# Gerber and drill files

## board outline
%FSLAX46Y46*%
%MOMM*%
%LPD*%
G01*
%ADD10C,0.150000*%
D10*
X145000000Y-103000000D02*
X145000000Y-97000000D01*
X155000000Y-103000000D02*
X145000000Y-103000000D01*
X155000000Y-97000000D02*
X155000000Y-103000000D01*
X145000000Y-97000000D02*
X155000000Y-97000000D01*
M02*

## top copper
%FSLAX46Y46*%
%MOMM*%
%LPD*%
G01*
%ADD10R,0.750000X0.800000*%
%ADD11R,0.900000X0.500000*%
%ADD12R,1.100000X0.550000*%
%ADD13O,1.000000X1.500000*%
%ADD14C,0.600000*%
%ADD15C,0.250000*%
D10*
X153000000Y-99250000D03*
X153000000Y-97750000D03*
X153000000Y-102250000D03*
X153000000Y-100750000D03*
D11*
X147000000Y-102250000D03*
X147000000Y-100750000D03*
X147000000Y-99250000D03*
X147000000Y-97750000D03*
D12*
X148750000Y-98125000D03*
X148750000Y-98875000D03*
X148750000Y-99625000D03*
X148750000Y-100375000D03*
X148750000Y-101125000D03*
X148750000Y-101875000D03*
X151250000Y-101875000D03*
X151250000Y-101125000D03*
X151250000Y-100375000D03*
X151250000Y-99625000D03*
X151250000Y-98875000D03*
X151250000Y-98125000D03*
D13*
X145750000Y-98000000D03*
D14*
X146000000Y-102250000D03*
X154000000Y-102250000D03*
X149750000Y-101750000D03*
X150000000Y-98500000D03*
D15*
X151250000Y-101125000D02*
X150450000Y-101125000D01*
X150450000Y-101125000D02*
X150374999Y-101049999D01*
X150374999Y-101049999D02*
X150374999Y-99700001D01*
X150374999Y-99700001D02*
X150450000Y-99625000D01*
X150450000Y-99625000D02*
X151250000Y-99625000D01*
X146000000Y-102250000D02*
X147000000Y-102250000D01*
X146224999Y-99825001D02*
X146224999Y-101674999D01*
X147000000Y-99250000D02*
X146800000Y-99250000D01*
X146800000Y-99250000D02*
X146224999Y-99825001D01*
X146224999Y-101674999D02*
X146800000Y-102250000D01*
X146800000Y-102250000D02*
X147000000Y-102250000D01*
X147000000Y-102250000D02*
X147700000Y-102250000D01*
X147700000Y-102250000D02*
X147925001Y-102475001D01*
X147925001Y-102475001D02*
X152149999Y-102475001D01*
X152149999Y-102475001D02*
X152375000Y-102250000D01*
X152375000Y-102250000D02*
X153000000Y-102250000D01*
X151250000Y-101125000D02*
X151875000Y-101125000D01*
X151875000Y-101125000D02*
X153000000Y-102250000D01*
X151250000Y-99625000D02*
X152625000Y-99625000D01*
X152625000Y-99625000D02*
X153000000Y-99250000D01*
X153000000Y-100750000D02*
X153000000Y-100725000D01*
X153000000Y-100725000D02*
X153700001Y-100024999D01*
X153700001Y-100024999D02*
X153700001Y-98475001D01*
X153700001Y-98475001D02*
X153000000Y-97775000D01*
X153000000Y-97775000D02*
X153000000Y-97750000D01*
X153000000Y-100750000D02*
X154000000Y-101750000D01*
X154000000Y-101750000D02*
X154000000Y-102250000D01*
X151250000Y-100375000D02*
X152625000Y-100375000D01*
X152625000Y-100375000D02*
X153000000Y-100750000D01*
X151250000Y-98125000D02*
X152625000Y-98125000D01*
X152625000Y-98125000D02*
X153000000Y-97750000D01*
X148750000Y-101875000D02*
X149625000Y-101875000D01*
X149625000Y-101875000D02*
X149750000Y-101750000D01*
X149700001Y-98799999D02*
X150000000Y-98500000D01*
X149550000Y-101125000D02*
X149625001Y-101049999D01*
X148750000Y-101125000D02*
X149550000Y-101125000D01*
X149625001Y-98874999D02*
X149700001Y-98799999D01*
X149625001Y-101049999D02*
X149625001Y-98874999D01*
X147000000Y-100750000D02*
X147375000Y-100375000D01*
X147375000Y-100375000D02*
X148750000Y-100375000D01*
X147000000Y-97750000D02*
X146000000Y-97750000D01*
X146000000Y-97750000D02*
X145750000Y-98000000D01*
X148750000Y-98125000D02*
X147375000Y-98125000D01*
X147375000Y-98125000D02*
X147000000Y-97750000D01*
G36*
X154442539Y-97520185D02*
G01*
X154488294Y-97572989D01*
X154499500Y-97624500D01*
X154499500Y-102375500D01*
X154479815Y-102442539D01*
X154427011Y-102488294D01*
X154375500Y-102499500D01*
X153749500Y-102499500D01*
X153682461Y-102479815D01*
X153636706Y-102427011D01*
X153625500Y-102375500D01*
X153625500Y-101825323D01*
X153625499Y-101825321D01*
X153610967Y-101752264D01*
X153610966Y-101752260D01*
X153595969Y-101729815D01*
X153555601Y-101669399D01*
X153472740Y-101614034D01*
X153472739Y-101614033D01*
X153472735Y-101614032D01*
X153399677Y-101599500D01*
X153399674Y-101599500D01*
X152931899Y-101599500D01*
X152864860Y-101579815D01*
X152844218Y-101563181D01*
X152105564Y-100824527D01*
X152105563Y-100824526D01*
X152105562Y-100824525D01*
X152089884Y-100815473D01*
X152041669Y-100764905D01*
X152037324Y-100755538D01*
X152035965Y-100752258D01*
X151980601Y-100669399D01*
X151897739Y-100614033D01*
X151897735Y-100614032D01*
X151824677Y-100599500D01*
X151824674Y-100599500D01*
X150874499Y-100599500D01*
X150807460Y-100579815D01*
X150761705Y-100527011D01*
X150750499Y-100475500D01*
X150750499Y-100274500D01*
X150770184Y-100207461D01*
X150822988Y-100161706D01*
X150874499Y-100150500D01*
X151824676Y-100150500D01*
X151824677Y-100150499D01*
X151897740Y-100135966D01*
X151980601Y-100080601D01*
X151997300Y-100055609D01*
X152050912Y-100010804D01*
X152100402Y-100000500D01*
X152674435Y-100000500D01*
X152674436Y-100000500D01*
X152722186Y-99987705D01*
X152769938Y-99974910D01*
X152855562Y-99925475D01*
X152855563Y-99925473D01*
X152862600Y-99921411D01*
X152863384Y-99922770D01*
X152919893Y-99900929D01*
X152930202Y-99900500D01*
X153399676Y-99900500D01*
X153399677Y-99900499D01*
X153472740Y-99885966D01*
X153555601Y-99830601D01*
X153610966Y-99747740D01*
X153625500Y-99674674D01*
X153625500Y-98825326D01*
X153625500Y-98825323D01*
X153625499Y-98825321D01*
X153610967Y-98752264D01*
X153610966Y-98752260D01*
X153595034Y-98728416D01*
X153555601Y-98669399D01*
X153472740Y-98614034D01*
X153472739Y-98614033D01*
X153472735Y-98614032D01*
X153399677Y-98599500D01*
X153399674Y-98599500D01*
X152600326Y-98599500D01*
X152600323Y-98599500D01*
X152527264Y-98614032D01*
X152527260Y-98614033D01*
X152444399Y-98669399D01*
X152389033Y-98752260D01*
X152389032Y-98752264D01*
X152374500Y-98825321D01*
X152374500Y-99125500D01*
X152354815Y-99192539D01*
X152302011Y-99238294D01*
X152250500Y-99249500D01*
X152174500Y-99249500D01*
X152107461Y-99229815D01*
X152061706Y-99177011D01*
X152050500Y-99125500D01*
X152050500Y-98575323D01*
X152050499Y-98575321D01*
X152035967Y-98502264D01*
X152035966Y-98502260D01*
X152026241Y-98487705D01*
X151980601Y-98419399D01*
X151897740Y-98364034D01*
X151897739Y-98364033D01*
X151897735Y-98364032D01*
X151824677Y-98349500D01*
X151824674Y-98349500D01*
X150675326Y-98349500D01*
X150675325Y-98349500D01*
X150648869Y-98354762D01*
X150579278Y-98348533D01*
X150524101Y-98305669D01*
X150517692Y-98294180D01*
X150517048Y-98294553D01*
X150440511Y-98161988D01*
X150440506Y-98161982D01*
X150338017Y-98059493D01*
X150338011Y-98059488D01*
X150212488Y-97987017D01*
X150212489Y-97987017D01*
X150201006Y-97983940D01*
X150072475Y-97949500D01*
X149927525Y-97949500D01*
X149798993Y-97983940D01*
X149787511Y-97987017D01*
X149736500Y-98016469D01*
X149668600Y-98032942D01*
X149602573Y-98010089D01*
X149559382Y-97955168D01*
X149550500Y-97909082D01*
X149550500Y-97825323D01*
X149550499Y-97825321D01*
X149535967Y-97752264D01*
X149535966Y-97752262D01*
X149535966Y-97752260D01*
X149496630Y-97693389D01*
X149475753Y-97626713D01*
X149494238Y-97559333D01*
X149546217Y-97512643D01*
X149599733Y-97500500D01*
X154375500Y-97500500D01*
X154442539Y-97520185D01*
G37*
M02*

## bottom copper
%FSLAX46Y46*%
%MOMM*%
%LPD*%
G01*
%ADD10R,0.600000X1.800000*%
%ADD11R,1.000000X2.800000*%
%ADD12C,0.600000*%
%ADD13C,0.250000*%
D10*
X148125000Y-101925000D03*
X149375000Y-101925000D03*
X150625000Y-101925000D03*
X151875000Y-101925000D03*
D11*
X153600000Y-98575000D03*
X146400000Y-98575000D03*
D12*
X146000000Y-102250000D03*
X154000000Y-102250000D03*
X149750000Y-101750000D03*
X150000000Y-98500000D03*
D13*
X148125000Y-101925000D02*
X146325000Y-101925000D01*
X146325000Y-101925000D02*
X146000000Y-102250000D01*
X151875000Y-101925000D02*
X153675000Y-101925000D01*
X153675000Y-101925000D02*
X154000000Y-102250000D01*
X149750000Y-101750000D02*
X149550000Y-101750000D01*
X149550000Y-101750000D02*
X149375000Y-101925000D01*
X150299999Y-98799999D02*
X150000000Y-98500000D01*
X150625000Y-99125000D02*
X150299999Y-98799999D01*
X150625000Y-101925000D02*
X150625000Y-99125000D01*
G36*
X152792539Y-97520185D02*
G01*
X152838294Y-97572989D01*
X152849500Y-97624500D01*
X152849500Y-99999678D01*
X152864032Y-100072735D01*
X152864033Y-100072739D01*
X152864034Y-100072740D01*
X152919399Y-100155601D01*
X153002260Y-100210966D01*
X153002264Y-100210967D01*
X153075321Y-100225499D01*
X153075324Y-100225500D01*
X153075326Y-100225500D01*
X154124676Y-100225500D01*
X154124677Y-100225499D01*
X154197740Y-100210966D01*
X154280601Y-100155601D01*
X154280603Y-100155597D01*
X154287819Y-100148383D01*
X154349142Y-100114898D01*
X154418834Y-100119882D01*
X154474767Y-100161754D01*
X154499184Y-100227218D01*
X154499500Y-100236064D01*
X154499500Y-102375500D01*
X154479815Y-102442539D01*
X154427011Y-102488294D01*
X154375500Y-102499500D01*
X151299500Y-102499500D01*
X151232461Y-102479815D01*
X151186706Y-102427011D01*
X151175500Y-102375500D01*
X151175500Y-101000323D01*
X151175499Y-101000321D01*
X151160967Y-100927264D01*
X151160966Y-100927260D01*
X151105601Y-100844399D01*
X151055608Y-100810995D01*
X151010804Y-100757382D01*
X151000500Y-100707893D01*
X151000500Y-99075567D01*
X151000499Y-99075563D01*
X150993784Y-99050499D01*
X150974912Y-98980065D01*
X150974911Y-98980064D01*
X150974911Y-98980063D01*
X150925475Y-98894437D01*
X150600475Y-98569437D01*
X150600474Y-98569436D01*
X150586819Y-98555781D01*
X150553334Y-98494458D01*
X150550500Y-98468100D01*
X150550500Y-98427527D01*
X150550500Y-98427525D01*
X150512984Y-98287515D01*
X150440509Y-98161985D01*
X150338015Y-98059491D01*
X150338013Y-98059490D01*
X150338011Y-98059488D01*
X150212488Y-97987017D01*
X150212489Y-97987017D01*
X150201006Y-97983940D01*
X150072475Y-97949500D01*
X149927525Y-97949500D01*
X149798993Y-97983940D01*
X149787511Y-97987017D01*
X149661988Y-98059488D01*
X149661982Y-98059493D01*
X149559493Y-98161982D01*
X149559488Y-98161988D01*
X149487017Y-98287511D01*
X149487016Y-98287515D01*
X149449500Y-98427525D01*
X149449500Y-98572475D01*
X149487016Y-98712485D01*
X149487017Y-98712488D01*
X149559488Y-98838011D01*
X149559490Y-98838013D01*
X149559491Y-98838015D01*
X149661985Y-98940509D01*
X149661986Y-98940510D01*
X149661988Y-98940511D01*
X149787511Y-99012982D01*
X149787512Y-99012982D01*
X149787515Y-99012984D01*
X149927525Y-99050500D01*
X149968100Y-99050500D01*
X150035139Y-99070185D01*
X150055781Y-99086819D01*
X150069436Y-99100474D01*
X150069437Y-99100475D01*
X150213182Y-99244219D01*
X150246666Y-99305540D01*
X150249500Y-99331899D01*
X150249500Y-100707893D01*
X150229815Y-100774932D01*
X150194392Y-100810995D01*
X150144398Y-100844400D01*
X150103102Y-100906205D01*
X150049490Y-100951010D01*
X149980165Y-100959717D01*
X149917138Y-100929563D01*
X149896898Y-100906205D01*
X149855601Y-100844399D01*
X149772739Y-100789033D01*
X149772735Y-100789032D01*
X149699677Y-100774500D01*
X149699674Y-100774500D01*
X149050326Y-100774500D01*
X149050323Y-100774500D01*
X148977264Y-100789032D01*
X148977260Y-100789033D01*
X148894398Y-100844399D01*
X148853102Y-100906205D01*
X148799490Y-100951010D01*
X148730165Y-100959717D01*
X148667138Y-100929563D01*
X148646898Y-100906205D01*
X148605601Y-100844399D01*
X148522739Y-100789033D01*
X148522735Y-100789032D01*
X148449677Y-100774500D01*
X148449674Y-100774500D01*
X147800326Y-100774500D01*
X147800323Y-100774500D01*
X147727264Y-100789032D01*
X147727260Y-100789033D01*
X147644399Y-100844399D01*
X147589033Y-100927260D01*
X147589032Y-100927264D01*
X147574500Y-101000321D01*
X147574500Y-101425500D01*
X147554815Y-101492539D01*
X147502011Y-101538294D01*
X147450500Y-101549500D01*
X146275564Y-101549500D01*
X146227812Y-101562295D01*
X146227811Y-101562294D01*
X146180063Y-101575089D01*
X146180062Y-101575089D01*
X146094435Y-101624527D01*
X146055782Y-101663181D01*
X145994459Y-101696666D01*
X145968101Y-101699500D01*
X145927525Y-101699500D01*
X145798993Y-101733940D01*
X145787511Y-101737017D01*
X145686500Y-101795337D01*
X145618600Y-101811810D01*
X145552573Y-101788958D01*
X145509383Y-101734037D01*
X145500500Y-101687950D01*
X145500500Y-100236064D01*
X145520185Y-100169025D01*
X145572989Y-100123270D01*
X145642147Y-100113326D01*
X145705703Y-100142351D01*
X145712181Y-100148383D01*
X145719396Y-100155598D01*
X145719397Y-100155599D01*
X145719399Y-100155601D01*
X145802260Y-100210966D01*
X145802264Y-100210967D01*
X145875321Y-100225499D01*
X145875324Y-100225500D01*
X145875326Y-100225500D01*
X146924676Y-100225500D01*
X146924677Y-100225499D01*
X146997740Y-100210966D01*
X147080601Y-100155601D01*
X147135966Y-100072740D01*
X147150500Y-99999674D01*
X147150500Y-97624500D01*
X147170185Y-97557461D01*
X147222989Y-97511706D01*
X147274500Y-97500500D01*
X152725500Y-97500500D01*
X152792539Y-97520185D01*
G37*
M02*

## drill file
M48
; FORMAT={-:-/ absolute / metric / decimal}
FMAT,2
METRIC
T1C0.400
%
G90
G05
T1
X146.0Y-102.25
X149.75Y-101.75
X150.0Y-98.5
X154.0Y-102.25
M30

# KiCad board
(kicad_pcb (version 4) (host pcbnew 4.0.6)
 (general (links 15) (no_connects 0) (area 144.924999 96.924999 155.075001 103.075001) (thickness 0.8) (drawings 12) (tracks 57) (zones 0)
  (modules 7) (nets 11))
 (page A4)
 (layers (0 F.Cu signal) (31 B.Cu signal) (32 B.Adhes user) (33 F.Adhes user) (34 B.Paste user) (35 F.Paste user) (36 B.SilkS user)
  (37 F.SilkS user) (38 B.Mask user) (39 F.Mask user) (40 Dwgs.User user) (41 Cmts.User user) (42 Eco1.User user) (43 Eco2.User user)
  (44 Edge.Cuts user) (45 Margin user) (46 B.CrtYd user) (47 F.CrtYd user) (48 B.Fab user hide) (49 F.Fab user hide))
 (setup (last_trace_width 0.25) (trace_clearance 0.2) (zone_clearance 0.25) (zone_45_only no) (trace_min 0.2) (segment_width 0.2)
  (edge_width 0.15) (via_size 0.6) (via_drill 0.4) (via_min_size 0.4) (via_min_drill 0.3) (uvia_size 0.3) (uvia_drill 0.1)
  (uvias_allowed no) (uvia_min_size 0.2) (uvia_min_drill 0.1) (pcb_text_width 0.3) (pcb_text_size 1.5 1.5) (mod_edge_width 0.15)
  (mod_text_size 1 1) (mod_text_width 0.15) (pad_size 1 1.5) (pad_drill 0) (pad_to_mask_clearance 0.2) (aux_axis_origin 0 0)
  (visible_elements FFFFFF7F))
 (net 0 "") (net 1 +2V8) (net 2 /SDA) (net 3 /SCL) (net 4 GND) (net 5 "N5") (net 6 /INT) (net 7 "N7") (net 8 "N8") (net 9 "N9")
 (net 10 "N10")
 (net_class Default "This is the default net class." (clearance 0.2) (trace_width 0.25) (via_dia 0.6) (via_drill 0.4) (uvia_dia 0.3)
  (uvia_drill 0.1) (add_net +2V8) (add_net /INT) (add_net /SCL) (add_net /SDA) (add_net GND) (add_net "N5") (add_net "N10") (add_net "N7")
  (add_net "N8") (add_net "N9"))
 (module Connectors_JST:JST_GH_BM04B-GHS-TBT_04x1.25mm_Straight (layer B.Cu) (at 150 100.25)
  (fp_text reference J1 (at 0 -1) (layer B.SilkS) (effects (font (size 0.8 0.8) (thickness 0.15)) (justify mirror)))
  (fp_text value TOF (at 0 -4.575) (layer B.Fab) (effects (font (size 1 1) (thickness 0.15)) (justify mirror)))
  (pad 1 smd rect (at -1.875 1.675) (size 0.6 1.8) (layers B.Cu B.Paste B.Mask) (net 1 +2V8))
  (pad 2 smd rect (at -0.625 1.675) (size 0.6 1.8) (layers B.Cu B.Paste B.Mask) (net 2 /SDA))
  (pad 3 smd rect (at 0.625 1.675) (size 0.6 1.8) (layers B.Cu B.Paste B.Mask) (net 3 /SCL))
  (pad 4 smd rect (at 1.875 1.675) (size 0.6 1.8) (layers B.Cu B.Paste B.Mask) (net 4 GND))
  (pad "" smd rect (at 3.6 -1.675) (size 1 2.8) (layers B.Cu B.Paste B.Mask))
  (pad "" smd rect (at -3.6 -1.675) (size 1 2.8) (layers B.Cu B.Paste B.Mask)))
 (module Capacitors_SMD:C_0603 (layer F.Cu) (at 153 98.5 90)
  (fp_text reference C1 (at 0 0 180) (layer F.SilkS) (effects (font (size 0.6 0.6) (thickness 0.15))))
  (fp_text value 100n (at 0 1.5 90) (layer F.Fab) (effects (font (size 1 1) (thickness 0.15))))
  (pad 1 smd rect (at -0.75 0 90) (size 0.8 0.75) (layers F.Cu F.Paste F.Mask) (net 1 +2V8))
  (pad 2 smd rect (at 0.75 0 90) (size 0.8 0.75) (layers F.Cu F.Paste F.Mask) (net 4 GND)))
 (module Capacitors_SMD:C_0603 (layer F.Cu) (at 153 101.5 90)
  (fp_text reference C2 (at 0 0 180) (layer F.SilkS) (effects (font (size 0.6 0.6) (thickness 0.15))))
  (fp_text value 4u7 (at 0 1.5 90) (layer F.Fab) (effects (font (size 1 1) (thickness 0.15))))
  (pad 1 smd rect (at -0.75 0 90) (size 0.8 0.75) (layers F.Cu F.Paste F.Mask) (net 1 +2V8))
  (pad 2 smd rect (at 0.75 0 90) (size 0.8 0.75) (layers F.Cu F.Paste F.Mask) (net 4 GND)))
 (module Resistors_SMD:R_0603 (layer F.Cu) (at 147 101.5 90)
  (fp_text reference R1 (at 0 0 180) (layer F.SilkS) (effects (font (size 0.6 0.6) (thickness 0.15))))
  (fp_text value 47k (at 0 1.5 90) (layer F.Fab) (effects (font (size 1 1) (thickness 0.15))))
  (pad 1 smd rect (at -0.75 0 90) (size 0.5 0.9) (layers F.Cu F.Paste F.Mask) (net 1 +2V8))
  (pad 2 smd rect (at 0.75 0 90) (size 0.5 0.9) (layers F.Cu F.Paste F.Mask) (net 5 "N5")))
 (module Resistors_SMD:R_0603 (layer F.Cu) (at 147 98.5 90)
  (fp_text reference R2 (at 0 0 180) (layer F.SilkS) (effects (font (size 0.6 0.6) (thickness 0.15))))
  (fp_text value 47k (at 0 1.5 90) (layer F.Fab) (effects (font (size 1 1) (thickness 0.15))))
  (pad 1 smd rect (at -0.75 0 90) (size 0.5 0.9) (layers F.Cu F.Paste F.Mask) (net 1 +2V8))
  (pad 2 smd rect (at 0.75 0 90) (size 0.5 0.9) (layers F.Cu F.Paste F.Mask) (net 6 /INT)))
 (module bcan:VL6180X (layer F.Cu) (at 150 100)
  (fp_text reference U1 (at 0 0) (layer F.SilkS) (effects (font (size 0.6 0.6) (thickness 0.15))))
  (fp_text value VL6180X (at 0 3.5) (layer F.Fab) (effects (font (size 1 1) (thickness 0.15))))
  (pad 1 smd rect (at -1.25 -1.875) (size 1.1 0.55) (layers F.Cu F.Paste F.Mask) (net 6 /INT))
  (pad 2 smd rect (at -1.25 -1.125) (size 1.1 0.55) (layers F.Cu F.Paste F.Mask) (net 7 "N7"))
  (pad 3 smd rect (at -1.25 -0.375) (size 1.1 0.55) (layers F.Cu F.Paste F.Mask) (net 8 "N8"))
  (pad 4 smd rect (at -1.25 0.375) (size 1.1 0.55) (layers F.Cu F.Paste F.Mask) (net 5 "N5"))
  (pad 5 smd rect (at -1.25 1.125) (size 1.1 0.55) (layers F.Cu F.Paste F.Mask) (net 3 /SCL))
  (pad 6 smd rect (at -1.25 1.875) (size 1.1 0.55) (layers F.Cu F.Paste F.Mask) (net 2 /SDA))
  (pad 7 smd rect (at 1.25 1.875) (size 1.1 0.55) (layers F.Cu F.Paste F.Mask) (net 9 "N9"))
  (pad 8 smd rect (at 1.25 1.125) (size 1.1 0.55) (layers F.Cu F.Paste F.Mask) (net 1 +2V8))
  (pad 9 smd rect (at 1.25 0.375) (size 1.1 0.55) (layers F.Cu F.Paste F.Mask) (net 4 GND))
  (pad 10 smd rect (at 1.25 -0.375) (size 1.1 0.55) (layers F.Cu F.Paste F.Mask) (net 1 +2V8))
  (pad 11 smd rect (at 1.25 -1.125) (size 1.1 0.55) (layers F.Cu F.Paste F.Mask) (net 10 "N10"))
  (pad 12 smd rect (at 1.25 -1.875) (size 1.1 0.55) (layers F.Cu F.Paste F.Mask) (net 4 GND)))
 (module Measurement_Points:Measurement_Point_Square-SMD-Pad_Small (layer F.Cu) (at 145.75 98)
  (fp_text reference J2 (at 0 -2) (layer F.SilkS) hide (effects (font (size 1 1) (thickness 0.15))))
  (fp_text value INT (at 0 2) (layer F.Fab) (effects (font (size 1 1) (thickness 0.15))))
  (pad 1 smd oval (at 0 0) (size 1 1.5) (layers F.Cu F.Mask) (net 6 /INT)))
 (gr_line (start 145 103) (end 145 97) (layer Edge.Cuts) (width 0.15))
 (gr_line (start 155 103) (end 145 103) (layer Edge.Cuts) (width 0.15))
 (gr_line (start 155 97) (end 155 103) (layer Edge.Cuts) (width 0.15))
 (gr_line (start 145 97) (end 155 97) (layer Edge.Cuts) (width 0.15))
 (segment (start 151.25 101.125) (end 150.45 101.125) (width 0.25) (layer F.Cu) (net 1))
 (segment (start 150.45 101.125) (end 150.374999 101.049999) (width 0.25) (layer F.Cu) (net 1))
 (segment (start 150.374999 101.049999) (end 150.374999 99.700001) (width 0.25) (layer F.Cu) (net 1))
 (segment (start 150.374999 99.700001) (end 150.45 99.625) (width 0.25) (layer F.Cu) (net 1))
 (segment (start 150.45 99.625) (end 151.25 99.625) (width 0.25) (layer F.Cu) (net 1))
 (segment (start 146 102.25) (end 147 102.25) (width 0.25) (layer F.Cu) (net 1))
 (segment (start 148.125 101.925) (end 146.325 101.925) (width 0.25) (layer B.Cu) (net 1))
 (segment (start 146.325 101.925) (end 146 102.25) (width 0.25) (layer B.Cu) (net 1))
 (via (at 146 102.25) (size 0.6) (drill 0.4) (layers F.Cu B.Cu) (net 1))
 (segment (start 146.224999 99.825001) (end 146.224999 101.674999) (width 0.25) (layer F.Cu) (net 1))
 (segment (start 147 99.25) (end 146.8 99.25) (width 0.25) (layer F.Cu) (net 1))
 (segment (start 146.8 99.25) (end 146.224999 99.825001) (width 0.25) (layer F.Cu) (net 1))
 (segment (start 146.224999 101.674999) (end 146.8 102.25) (width 0.25) (layer F.Cu) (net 1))
 (segment (start 146.8 102.25) (end 147 102.25) (width 0.25) (layer F.Cu) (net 1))
 (segment (start 147 102.25) (end 147.7 102.25) (width 0.25) (layer F.Cu) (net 1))
 (segment (start 147.7 102.25) (end 147.925001 102.475001) (width 0.25) (layer F.Cu) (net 1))
 (segment (start 147.925001 102.475001) (end 152.149999 102.475001) (width 0.25) (layer F.Cu) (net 1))
 (segment (start 152.149999 102.475001) (end 152.375 102.25) (width 0.25) (layer F.Cu) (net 1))
 (segment (start 152.375 102.25) (end 153 102.25) (width 0.25) (layer F.Cu) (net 1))
 (segment (start 151.25 101.125) (end 151.875 101.125) (width 0.25) (layer F.Cu) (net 1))
 (segment (start 151.875 101.125) (end 153 102.25) (width 0.25) (layer F.Cu) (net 1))
 (segment (start 151.25 99.625) (end 152.625 99.625) (width 0.25) (layer F.Cu) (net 1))
 (segment (start 152.625 99.625) (end 153 99.25) (width 0.25) (layer F.Cu) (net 1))
 (segment (start 153 100.75) (end 153 100.725) (width 0.25) (layer F.Cu) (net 4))
 (segment (start 153 100.725) (end 153.700001 100.024999) (width 0.25) (layer F.Cu) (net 4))
 (segment (start 153.700001 100.024999) (end 153.700001 98.475001) (width 0.25) (layer F.Cu) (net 4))
 (segment (start 153.700001 98.475001) (end 153 97.775) (width 0.25) (layer F.Cu) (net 4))
 (segment (start 153 97.775) (end 153 97.75) (width 0.25) (layer F.Cu) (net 4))
 (segment (start 151.875 101.925) (end 153.675 101.925) (width 0.25) (layer B.Cu) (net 4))
 (segment (start 153.675 101.925) (end 154 102.25) (width 0.25) (layer B.Cu) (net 4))
 (segment (start 153 100.75) (end 154 101.75) (width 0.25) (layer F.Cu) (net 4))
 (via (at 154 102.25) (size 0.6) (drill 0.4) (layers F.Cu B.Cu) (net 4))
 (segment (start 154 101.75) (end 154 102.25) (width 0.25) (layer F.Cu) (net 4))
 (segment (start 151.25 100.375) (end 152.625 100.375) (width 0.25) (layer F.Cu) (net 4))
 (segment (start 152.625 100.375) (end 153 100.75) (width 0.25) (layer F.Cu) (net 4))
 (segment (start 151.25 98.125) (end 152.625 98.125) (width 0.25) (layer F.Cu) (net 4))
 (segment (start 152.625 98.125) (end 153 97.75) (width 0.25) (layer F.Cu) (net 4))
 (segment (start 149.75 101.75) (end 149.55 101.75) (width 0.25) (layer B.Cu) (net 2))
 (segment (start 149.55 101.75) (end 149.375 101.925) (width 0.25) (layer B.Cu) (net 2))
 (segment (start 148.75 101.875) (end 149.625 101.875) (width 0.25) (layer F.Cu) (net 2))
 (segment (start 149.625 101.875) (end 149.75 101.75) (width 0.25) (layer F.Cu) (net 2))
 (via (at 149.75 101.75) (size 0.6) (drill 0.4) (layers F.Cu B.Cu) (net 2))
 (segment (start 149.700001 98.799999) (end 150 98.5) (width 0.25) (layer F.Cu) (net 3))
 (segment (start 149.55 101.125) (end 149.625001 101.049999) (width 0.25) (layer F.Cu) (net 3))
 (segment (start 148.75 101.125) (end 149.55 101.125) (width 0.25) (layer F.Cu) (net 3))
 (segment (start 149.625001 98.874999) (end 149.700001 98.799999) (width 0.25) (layer F.Cu) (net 3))
 (segment (start 149.625001 101.049999) (end 149.625001 98.874999) (width 0.25) (layer F.Cu) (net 3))
 (segment (start 150.299999 98.799999) (end 150 98.5) (width 0.25) (layer B.Cu) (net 3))
 (segment (start 150.625 99.125) (end 150.299999 98.799999) (width 0.25) (layer B.Cu) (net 3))
 (segment (start 150.625 101.925) (end 150.625 99.125) (width 0.25) (layer B.Cu) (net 3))
 (via (at 150 98.5) (size 0.6) (drill 0.4) (layers F.Cu B.Cu) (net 3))
 (segment (start 147 100.75) (end 147.375 100.375) (width 0.25) (layer F.Cu) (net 5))
 (segment (start 147.375 100.375) (end 148.75 100.375) (width 0.25) (layer F.Cu) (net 5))
 (segment (start 147 97.75) (end 146 97.75) (width 0.25) (layer F.Cu) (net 6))
 (segment (start 146 97.75) (end 145.75 98) (width 0.25) (layer F.Cu) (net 6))
 (segment (start 148.75 98.125) (end 147.375 98.125) (width 0.25) (layer F.Cu) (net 6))
 (segment (start 147.375 98.125) (end 147 97.75) (width 0.25) (layer F.Cu) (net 6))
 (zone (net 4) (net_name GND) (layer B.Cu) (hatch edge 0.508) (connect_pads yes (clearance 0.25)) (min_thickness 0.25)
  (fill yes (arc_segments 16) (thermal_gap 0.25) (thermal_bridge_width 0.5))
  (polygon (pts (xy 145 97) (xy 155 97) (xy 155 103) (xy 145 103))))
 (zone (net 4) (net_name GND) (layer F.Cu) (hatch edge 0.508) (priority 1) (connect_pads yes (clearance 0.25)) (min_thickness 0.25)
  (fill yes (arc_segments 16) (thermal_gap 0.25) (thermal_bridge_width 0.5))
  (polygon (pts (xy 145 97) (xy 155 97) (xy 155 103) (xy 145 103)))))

